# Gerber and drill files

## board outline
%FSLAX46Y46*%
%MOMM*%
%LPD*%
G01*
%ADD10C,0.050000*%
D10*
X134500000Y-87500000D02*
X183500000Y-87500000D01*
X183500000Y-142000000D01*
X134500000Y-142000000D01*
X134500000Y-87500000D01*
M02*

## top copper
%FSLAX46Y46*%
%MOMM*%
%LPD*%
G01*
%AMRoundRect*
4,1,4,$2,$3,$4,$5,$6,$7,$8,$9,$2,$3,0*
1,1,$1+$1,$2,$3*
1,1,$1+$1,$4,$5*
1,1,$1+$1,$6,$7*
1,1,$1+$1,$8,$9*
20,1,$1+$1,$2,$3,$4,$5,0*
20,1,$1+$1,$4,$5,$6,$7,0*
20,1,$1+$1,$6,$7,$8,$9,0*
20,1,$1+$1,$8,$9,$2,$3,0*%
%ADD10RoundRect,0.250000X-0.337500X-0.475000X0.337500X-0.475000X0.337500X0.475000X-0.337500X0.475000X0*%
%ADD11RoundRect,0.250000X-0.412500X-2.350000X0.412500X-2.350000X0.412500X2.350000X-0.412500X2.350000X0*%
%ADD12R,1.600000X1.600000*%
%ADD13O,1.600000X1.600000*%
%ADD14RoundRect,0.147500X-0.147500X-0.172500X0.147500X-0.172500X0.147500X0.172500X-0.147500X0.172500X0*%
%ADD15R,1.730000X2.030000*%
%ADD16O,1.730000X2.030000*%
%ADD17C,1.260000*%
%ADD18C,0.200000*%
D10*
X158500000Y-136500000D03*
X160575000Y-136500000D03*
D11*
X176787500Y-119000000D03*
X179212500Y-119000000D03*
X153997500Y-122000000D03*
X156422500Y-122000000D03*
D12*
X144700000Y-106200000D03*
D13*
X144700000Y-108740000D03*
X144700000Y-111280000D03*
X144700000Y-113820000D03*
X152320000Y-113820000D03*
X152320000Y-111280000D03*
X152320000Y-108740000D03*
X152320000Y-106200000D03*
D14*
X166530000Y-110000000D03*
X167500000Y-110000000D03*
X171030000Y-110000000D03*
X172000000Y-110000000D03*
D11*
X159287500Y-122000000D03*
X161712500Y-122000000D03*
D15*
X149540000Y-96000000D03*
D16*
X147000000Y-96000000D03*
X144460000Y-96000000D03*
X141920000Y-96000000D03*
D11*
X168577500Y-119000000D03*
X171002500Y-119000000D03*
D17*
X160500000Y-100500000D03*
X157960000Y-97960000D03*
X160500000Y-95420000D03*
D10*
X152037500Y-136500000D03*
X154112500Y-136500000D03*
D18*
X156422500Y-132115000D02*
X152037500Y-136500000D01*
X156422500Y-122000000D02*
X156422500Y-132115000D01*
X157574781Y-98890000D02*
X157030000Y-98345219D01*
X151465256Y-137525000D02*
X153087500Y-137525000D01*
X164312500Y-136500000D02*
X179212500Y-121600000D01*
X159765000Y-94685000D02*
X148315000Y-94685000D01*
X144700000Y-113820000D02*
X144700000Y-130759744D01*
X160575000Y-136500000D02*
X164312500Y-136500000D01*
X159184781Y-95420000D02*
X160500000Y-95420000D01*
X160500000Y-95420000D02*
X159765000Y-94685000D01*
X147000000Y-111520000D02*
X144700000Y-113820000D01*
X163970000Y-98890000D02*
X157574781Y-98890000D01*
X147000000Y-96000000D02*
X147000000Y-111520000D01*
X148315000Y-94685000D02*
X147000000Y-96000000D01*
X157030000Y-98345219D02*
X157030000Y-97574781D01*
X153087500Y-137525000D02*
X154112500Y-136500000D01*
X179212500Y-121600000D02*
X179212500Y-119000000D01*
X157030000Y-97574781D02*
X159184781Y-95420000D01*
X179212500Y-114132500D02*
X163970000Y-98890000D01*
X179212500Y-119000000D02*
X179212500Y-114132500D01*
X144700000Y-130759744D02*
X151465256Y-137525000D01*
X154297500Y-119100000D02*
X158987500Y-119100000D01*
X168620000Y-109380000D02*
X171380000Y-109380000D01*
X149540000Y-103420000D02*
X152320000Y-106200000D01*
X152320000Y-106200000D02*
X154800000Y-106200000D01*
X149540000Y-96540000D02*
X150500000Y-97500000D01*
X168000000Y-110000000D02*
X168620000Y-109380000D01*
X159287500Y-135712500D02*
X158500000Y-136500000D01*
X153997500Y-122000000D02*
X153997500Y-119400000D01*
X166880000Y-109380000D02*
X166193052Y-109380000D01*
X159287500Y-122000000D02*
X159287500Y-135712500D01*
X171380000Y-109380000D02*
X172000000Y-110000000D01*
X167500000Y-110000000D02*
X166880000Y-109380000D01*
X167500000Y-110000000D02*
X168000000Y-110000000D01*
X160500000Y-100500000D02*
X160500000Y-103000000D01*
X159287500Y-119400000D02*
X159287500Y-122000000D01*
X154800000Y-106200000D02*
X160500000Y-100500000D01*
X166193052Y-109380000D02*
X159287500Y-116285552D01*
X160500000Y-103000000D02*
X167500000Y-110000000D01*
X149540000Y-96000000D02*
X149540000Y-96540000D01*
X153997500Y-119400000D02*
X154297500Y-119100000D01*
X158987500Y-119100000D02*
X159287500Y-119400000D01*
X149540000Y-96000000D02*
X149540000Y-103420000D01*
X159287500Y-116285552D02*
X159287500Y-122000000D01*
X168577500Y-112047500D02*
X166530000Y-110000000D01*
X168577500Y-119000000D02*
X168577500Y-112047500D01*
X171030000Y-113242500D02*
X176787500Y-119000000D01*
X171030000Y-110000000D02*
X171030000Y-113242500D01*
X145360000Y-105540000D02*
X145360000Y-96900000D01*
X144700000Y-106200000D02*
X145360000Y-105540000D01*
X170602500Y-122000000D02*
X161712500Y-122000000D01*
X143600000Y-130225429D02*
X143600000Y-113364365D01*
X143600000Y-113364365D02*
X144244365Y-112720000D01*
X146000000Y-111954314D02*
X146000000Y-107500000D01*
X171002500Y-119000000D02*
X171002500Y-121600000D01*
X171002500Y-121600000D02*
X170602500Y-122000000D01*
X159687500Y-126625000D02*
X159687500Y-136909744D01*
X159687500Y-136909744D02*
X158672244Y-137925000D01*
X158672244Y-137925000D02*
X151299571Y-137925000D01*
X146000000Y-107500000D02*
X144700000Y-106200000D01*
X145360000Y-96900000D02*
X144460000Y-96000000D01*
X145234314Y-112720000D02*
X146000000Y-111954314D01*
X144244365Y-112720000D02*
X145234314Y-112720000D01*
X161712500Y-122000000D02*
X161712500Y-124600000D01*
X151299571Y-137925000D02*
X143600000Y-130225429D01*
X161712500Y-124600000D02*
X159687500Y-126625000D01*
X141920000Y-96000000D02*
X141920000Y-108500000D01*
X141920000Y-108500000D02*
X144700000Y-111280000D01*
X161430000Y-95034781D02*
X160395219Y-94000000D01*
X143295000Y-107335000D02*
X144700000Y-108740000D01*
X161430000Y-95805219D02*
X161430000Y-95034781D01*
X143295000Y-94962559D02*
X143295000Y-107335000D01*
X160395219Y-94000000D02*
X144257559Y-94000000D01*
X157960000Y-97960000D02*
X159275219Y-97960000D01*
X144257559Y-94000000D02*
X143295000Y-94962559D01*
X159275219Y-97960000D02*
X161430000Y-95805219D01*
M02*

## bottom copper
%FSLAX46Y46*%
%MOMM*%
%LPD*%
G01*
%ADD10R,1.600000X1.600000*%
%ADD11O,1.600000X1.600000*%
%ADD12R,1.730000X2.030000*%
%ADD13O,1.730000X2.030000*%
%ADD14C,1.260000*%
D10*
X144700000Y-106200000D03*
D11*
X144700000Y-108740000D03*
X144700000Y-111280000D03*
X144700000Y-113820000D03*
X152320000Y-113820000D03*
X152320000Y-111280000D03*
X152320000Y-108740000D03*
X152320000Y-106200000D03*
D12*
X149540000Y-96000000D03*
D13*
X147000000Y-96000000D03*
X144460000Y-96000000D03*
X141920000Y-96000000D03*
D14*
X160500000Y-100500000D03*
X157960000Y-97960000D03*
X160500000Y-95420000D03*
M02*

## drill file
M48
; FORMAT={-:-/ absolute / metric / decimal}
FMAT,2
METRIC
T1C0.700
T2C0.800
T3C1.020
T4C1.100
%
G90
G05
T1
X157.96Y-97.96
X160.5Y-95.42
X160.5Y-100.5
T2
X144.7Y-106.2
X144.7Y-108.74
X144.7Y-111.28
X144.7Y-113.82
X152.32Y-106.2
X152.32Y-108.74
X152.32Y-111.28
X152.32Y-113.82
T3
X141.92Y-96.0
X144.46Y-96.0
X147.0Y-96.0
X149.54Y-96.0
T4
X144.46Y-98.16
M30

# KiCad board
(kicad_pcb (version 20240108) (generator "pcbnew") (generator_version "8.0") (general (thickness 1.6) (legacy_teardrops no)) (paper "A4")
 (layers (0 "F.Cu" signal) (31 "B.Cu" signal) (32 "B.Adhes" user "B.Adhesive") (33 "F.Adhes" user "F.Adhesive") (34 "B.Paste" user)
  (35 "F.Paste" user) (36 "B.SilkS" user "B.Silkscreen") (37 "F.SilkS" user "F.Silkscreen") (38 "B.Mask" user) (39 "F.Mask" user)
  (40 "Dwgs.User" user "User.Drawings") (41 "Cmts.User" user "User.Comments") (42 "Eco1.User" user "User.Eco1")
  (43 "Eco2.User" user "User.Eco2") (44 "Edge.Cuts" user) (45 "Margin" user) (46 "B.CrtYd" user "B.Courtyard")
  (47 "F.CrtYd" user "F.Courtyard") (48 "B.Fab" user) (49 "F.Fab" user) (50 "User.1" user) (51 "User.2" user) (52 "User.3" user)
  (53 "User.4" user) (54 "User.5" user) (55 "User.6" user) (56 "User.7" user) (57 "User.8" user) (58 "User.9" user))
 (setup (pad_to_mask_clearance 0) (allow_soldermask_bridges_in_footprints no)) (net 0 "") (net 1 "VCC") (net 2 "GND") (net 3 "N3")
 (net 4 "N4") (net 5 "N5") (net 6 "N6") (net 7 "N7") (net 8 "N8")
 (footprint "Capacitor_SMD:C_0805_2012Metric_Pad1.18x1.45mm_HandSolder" (layer "F.Cu") (at 159.5375 136.5)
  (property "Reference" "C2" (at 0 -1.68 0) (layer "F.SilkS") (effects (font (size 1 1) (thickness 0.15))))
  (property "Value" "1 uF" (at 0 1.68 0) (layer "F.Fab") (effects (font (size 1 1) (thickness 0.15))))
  (pad "1" smd roundrect (at -1.0375 0) (size 1.175 1.45) (layers "F.Cu" "F.Paste" "F.Mask") (roundrect_rratio 0.212766) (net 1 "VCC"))
  (pad "2" smd roundrect (at 1.0375 0) (size 1.175 1.45) (layers "F.Cu" "F.Paste" "F.Mask") (roundrect_rratio 0.212766) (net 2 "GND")))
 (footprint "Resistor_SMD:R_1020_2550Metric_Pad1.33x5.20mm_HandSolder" (layer "F.Cu") (at 178 119)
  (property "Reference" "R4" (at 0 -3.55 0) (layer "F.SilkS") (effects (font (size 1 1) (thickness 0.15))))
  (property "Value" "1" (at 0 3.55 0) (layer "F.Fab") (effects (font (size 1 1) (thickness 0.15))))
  (pad "1" smd roundrect (at -1.2125 0) (size 1.325 5.2) (layers "F.Cu" "F.Paste" "F.Mask") (roundrect_rratio 0.188679) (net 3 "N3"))
  (pad "2" smd roundrect (at 1.2125 0) (size 1.325 5.2) (layers "F.Cu" "F.Paste" "F.Mask") (roundrect_rratio 0.188679) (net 2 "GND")))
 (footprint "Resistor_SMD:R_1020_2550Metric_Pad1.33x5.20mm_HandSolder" (layer "F.Cu") (at 155.21 122)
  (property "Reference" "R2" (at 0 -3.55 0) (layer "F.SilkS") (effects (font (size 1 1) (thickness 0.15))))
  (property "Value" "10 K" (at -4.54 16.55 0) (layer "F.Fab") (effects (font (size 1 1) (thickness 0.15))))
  (pad "1" smd roundrect (at -1.2125 0) (size 1.325 5.2) (layers "F.Cu" "F.Paste" "F.Mask") (roundrect_rratio 0.188679) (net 1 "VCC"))
  (pad "2" smd roundrect (at 1.2125 0) (size 1.325 5.2) (layers "F.Cu" "F.Paste" "F.Mask") (roundrect_rratio 0.188679) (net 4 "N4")))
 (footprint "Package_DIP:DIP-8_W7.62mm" (layer "F.Cu") (at 144.7 106.2)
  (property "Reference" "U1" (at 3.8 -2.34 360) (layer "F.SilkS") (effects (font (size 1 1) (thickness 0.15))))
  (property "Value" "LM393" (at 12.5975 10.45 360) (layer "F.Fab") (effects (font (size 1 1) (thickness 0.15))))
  (pad "1" thru_hole rect (at 0 0) (size 1.6 1.6) (drill 0.8) (layers "*.Cu" "*.Mask") (remove_unused_layers no) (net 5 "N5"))
  (pad "2" thru_hole oval (at 0 2.54) (size 1.6 1.6) (drill 0.8) (layers "*.Cu" "*.Mask") (remove_unused_layers no) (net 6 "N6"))
  (pad "3" thru_hole oval (at 0 5.08) (size 1.6 1.6) (drill 0.8) (layers "*.Cu" "*.Mask") (remove_unused_layers no) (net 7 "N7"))
  (pad "4" thru_hole oval (at 0 7.62) (size 1.6 1.6) (drill 0.8) (layers "*.Cu" "*.Mask") (remove_unused_layers no) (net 2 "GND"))
  (pad "5" thru_hole oval (at 7.62 7.62) (size 1.6 1.6) (drill 0.8) (layers "*.Cu" "*.Mask") (remove_unused_layers no))
  (pad "6" thru_hole oval (at 7.62 5.08) (size 1.6 1.6) (drill 0.8) (layers "*.Cu" "*.Mask") (remove_unused_layers no))
  (pad "7" thru_hole oval (at 7.62 2.54) (size 1.6 1.6) (drill 0.8) (layers "*.Cu" "*.Mask") (remove_unused_layers no))
  (pad "8" thru_hole oval (at 7.62 0) (size 1.6 1.6) (drill 0.8) (layers "*.Cu" "*.Mask") (remove_unused_layers no) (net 1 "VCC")))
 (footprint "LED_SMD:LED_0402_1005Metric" (layer "F.Cu") (at 167.015 110)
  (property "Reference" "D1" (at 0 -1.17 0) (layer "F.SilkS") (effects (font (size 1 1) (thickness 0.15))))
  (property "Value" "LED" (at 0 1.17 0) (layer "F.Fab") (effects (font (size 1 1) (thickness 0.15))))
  (pad "1" smd roundrect (at -0.485 0) (size 0.59 0.64) (layers "F.Cu" "F.Paste" "F.Mask") (roundrect_rratio 0.25) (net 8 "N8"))
  (pad "2" smd roundrect (at 0.485 0) (size 0.59 0.64) (layers "F.Cu" "F.Paste" "F.Mask") (roundrect_rratio 0.25) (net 1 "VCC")))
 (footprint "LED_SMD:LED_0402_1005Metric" (layer "F.Cu") (at 171.515 110)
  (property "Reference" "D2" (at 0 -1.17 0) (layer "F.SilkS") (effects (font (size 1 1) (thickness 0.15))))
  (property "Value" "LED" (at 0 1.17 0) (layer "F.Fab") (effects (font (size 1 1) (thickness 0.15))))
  (pad "1" smd roundrect (at -0.485 0) (size 0.59 0.64) (layers "F.Cu" "F.Paste" "F.Mask") (roundrect_rratio 0.25) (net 3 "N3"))
  (pad "2" smd roundrect (at 0.485 0) (size 0.59 0.64) (layers "F.Cu" "F.Paste" "F.Mask") (roundrect_rratio 0.25) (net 1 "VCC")))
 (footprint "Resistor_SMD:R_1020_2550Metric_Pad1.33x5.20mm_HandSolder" (layer "F.Cu") (at 160.5 122)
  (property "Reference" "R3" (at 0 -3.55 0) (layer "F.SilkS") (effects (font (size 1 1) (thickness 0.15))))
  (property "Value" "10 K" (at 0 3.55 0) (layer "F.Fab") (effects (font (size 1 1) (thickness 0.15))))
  (pad "1" smd roundrect (at -1.2125 0) (size 1.325 5.2) (layers "F.Cu" "F.Paste" "F.Mask") (roundrect_rratio 0.188679) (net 1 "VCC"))
  (pad "2" smd roundrect (at 1.2125 0) (size 1.325 5.2) (layers "F.Cu" "F.Paste" "F.Mask") (roundrect_rratio 0.188679) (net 5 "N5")))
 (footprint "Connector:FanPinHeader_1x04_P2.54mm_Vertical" (layer "F.Cu") (at 149.54 96 180)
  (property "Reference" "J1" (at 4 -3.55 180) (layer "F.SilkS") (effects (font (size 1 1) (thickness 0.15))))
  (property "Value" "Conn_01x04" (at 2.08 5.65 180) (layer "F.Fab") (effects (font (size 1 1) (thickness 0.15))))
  (pad "" np_thru_hole circle (at 5.08 -2.16 270) (size 1.1 1.1) (drill 1.1) (layers "*.Cu" "*.Mask"))
  (pad "1" thru_hole rect (at 0 0 270) (size 2.03 1.73) (drill 1.02) (layers "*.Cu" "*.Mask") (remove_unused_layers no) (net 1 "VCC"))
  (pad "2" thru_hole oval (at 2.54 0 270) (size 2.03 1.73) (drill 1.02) (layers "*.Cu" "*.Mask") (remove_unused_layers no) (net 2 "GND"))
  (pad "3" thru_hole oval (at 5.08 0 270) (size 2.03 1.73) (drill 1.02) (layers "*.Cu" "*.Mask") (remove_unused_layers no) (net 5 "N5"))
  (pad "4" thru_hole oval (at 7.62 0 270) (size 2.03 1.73) (drill 1.02) (layers "*.Cu" "*.Mask") (remove_unused_layers no) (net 7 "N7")))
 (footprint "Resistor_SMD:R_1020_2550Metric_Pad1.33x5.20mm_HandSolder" (layer "F.Cu") (at 169.79 119)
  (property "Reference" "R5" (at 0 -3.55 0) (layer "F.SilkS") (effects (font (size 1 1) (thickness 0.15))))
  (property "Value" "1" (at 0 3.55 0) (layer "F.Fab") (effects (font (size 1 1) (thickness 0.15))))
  (pad "1" smd roundrect (at -1.2125 0) (size 1.325 5.2) (layers "F.Cu" "F.Paste" "F.Mask") (roundrect_rratio 0.188679) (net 8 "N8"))
  (pad "2" smd roundrect (at 1.2125 0) (size 1.325 5.2) (layers "F.Cu" "F.Paste" "F.Mask") (roundrect_rratio 0.188679) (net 5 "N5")))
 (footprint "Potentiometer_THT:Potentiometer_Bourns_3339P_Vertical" (layer "F.Cu") (at 160.5 100.5)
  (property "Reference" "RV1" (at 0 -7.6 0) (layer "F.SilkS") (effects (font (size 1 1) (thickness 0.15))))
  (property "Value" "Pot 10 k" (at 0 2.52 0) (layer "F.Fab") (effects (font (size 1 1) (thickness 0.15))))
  (pad "1" thru_hole circle (at 0 0) (size 1.26 1.26) (drill 0.7) (layers "*.Cu" "*.Mask") (remove_unused_layers no) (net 1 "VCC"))
  (pad "2" thru_hole circle (at -2.54 -2.54) (size 1.26 1.26) (drill 0.7) (layers "*.Cu" "*.Mask") (remove_unused_layers no) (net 6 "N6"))
  (pad "3" thru_hole circle (at 0 -5.08) (size 1.26 1.26) (drill 0.7) (layers "*.Cu" "*.Mask") (remove_unused_layers no) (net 2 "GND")))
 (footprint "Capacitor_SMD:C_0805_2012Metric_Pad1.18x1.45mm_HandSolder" (layer "F.Cu") (at 153.075 136.5)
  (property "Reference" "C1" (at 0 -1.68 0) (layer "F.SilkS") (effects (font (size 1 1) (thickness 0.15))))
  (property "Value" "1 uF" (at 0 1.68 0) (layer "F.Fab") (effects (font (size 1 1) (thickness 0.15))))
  (pad "1" smd roundrect (at -1.0375 0) (size 1.175 1.45) (layers "F.Cu" "F.Paste" "F.Mask") (roundrect_rratio 0.212766) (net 4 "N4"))
  (pad "2" smd roundrect (at 1.0375 0) (size 1.175 1.45) (layers "F.Cu" "F.Paste" "F.Mask") (roundrect_rratio 0.212766) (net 2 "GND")))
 (gr_rect (start 134.5 87.5) (end 183.5 142) (stroke (width 0.05) (type default)) (fill none) (layer "Edge.Cuts"))
 (segment (start 156.4225 132.115) (end 152.0375 136.5) (width 0.2) (layer "F.Cu") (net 4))
 (segment (start 156.4225 122) (end 156.4225 132.115) (width 0.2) (layer "F.Cu") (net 4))
 (segment (start 157.574781 98.89) (end 157.03 98.345219) (width 0.2) (layer "F.Cu") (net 2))
 (segment (start 151.465256 137.525) (end 153.0875 137.525) (width 0.2) (layer "F.Cu") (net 2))
 (segment (start 164.3125 136.5) (end 179.2125 121.6) (width 0.2) (layer "F.Cu") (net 2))
 (segment (start 159.765 94.685) (end 148.315 94.685) (width 0.2) (layer "F.Cu") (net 2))
 (segment (start 144.7 113.82) (end 144.7 130.759744) (width 0.2) (layer "F.Cu") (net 2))
 (segment (start 160.575 136.5) (end 164.3125 136.5) (width 0.2) (layer "F.Cu") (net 2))
 (segment (start 159.184781 95.42) (end 160.5 95.42) (width 0.2) (layer "F.Cu") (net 2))
 (segment (start 160.5 95.42) (end 159.765 94.685) (width 0.2) (layer "F.Cu") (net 2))
 (segment (start 147 111.52) (end 144.7 113.82) (width 0.2) (layer "F.Cu") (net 2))
 (segment (start 163.97 98.89) (end 157.574781 98.89) (width 0.2) (layer "F.Cu") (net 2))
 (segment (start 147 96) (end 147 111.52) (width 0.2) (layer "F.Cu") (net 2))
 (segment (start 148.315 94.685) (end 147 96) (width 0.2) (layer "F.Cu") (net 2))
 (segment (start 157.03 98.345219) (end 157.03 97.574781) (width 0.2) (layer "F.Cu") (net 2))
 (segment (start 153.0875 137.525) (end 154.1125 136.5) (width 0.2) (layer "F.Cu") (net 2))
 (segment (start 179.2125 121.6) (end 179.2125 119) (width 0.2) (layer "F.Cu") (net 2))
 (segment (start 157.03 97.574781) (end 159.184781 95.42) (width 0.2) (layer "F.Cu") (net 2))
 (segment (start 179.2125 114.1325) (end 163.97 98.89) (width 0.2) (layer "F.Cu") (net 2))
 (segment (start 179.2125 119) (end 179.2125 114.1325) (width 0.2) (layer "F.Cu") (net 2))
 (segment (start 144.7 130.759744) (end 151.465256 137.525) (width 0.2) (layer "F.Cu") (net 2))
 (segment (start 154.2975 119.1) (end 158.9875 119.1) (width 0.2) (layer "F.Cu") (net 1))
 (segment (start 168.62 109.38) (end 171.38 109.38) (width 0.2) (layer "F.Cu") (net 1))
 (segment (start 149.54 103.42) (end 152.32 106.2) (width 0.2) (layer "F.Cu") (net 1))
 (segment (start 152.32 106.2) (end 154.8 106.2) (width 0.2) (layer "F.Cu") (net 1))
 (segment (start 149.54 96.54) (end 150.5 97.5) (width 0.2) (layer "F.Cu") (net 1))
 (segment (start 168 110) (end 168.62 109.38) (width 0.2) (layer "F.Cu") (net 1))
 (segment (start 159.2875 135.7125) (end 158.5 136.5) (width 0.2) (layer "F.Cu") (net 1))
 (segment (start 153.9975 122) (end 153.9975 119.4) (width 0.2) (layer "F.Cu") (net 1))
 (segment (start 166.88 109.38) (end 166.193052 109.38) (width 0.2) (layer "F.Cu") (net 1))
 (segment (start 159.2875 122) (end 159.2875 135.7125) (width 0.2) (layer "F.Cu") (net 1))
 (segment (start 171.38 109.38) (end 172 110) (width 0.2) (layer "F.Cu") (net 1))
 (segment (start 167.5 110) (end 166.88 109.38) (width 0.2) (layer "F.Cu") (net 1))
 (segment (start 167.5 110) (end 168 110) (width 0.2) (layer "F.Cu") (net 1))
 (segment (start 160.5 100.5) (end 160.5 103) (width 0.2) (layer "F.Cu") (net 1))
 (segment (start 159.2875 119.4) (end 159.2875 122) (width 0.2) (layer "F.Cu") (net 1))
 (segment (start 154.8 106.2) (end 160.5 100.5) (width 0.2) (layer "F.Cu") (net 1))
 (segment (start 166.193052 109.38) (end 159.2875 116.285552) (width 0.2) (layer "F.Cu") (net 1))
 (segment (start 160.5 103) (end 167.5 110) (width 0.2) (layer "F.Cu") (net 1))
 (segment (start 149.54 96) (end 149.54 96.54) (width 0.2) (layer "F.Cu") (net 1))
 (segment (start 153.9975 119.4) (end 154.2975 119.1) (width 0.2) (layer "F.Cu") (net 1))
 (segment (start 158.9875 119.1) (end 159.2875 119.4) (width 0.2) (layer "F.Cu") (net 1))
 (segment (start 149.54 96) (end 149.54 103.42) (width 0.2) (layer "F.Cu") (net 1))
 (segment (start 159.2875 116.285552) (end 159.2875 122) (width 0.2) (layer "F.Cu") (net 1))
 (segment (start 168.5775 112.0475) (end 166.53 110) (width 0.2) (layer "F.Cu") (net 8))
 (segment (start 168.5775 119) (end 168.5775 112.0475) (width 0.2) (layer "F.Cu") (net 8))
 (segment (start 171.03 113.2425) (end 176.7875 119) (width 0.2) (layer "F.Cu") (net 3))
 (segment (start 171.03 110) (end 171.03 113.2425) (width 0.2) (layer "F.Cu") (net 3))
 (segment (start 145.36 105.54) (end 145.36 96.9) (width 0.2) (layer "F.Cu") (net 5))
 (segment (start 144.7 106.2) (end 145.36 105.54) (width 0.2) (layer "F.Cu") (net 5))
 (segment (start 170.6025 122) (end 161.7125 122) (width 0.2) (layer "F.Cu") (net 5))
 (segment (start 143.6 130.225429) (end 143.6 113.364365) (width 0.2) (layer "F.Cu") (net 5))
 (segment (start 143.6 113.364365) (end 144.244365 112.72) (width 0.2) (layer "F.Cu") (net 5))
 (segment (start 146 111.954314) (end 146 107.5) (width 0.2) (layer "F.Cu") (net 5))
 (segment (start 171.0025 119) (end 171.0025 121.6) (width 0.2) (layer "F.Cu") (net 5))
 (segment (start 171.0025 121.6) (end 170.6025 122) (width 0.2) (layer "F.Cu") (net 5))
 (segment (start 159.6875 126.625) (end 159.6875 136.909744) (width 0.2) (layer "F.Cu") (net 5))
 (segment (start 159.6875 136.909744) (end 158.672244 137.925) (width 0.2) (layer "F.Cu") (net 5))
 (segment (start 158.672244 137.925) (end 151.299571 137.925) (width 0.2) (layer "F.Cu") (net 5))
 (segment (start 146 107.5) (end 144.7 106.2) (width 0.2) (layer "F.Cu") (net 5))
 (segment (start 145.36 96.9) (end 144.46 96) (width 0.2) (layer "F.Cu") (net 5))
 (segment (start 145.234314 112.72) (end 146 111.954314) (width 0.2) (layer "F.Cu") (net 5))
 (segment (start 144.244365 112.72) (end 145.234314 112.72) (width 0.2) (layer "F.Cu") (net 5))
 (segment (start 161.7125 122) (end 161.7125 124.6) (width 0.2) (layer "F.Cu") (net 5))
 (segment (start 151.299571 137.925) (end 143.6 130.225429) (width 0.2) (layer "F.Cu") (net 5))
 (segment (start 161.7125 124.6) (end 159.6875 126.625) (width 0.2) (layer "F.Cu") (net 5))
 (segment (start 141.92 96) (end 141.92 108.5) (width 0.2) (layer "F.Cu") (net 7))
 (segment (start 141.92 108.5) (end 144.7 111.28) (width 0.2) (layer "F.Cu") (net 7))
 (segment (start 161.43 95.034781) (end 160.395219 94) (width 0.2) (layer "F.Cu") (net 6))
 (segment (start 143.295 107.335) (end 144.7 108.74) (width 0.2) (layer "F.Cu") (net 6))
 (segment (start 161.43 95.805219) (end 161.43 95.034781) (width 0.2) (layer "F.Cu") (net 6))
 (segment (start 143.295 94.962559) (end 143.295 107.335) (width 0.2) (layer "F.Cu") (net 6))
 (segment (start 160.395219 94) (end 144.257559 94) (width 0.2) (layer "F.Cu") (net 6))
 (segment (start 157.96 97.96) (end 159.275219 97.96) (width 0.2) (layer "F.Cu") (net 6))
 (segment (start 144.257559 94) (end 143.295 94.962559) (width 0.2) (layer "F.Cu") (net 6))
 (segment (start 159.275219 97.96) (end 161.43 95.805219) (width 0.2) (layer "F.Cu") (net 6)))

